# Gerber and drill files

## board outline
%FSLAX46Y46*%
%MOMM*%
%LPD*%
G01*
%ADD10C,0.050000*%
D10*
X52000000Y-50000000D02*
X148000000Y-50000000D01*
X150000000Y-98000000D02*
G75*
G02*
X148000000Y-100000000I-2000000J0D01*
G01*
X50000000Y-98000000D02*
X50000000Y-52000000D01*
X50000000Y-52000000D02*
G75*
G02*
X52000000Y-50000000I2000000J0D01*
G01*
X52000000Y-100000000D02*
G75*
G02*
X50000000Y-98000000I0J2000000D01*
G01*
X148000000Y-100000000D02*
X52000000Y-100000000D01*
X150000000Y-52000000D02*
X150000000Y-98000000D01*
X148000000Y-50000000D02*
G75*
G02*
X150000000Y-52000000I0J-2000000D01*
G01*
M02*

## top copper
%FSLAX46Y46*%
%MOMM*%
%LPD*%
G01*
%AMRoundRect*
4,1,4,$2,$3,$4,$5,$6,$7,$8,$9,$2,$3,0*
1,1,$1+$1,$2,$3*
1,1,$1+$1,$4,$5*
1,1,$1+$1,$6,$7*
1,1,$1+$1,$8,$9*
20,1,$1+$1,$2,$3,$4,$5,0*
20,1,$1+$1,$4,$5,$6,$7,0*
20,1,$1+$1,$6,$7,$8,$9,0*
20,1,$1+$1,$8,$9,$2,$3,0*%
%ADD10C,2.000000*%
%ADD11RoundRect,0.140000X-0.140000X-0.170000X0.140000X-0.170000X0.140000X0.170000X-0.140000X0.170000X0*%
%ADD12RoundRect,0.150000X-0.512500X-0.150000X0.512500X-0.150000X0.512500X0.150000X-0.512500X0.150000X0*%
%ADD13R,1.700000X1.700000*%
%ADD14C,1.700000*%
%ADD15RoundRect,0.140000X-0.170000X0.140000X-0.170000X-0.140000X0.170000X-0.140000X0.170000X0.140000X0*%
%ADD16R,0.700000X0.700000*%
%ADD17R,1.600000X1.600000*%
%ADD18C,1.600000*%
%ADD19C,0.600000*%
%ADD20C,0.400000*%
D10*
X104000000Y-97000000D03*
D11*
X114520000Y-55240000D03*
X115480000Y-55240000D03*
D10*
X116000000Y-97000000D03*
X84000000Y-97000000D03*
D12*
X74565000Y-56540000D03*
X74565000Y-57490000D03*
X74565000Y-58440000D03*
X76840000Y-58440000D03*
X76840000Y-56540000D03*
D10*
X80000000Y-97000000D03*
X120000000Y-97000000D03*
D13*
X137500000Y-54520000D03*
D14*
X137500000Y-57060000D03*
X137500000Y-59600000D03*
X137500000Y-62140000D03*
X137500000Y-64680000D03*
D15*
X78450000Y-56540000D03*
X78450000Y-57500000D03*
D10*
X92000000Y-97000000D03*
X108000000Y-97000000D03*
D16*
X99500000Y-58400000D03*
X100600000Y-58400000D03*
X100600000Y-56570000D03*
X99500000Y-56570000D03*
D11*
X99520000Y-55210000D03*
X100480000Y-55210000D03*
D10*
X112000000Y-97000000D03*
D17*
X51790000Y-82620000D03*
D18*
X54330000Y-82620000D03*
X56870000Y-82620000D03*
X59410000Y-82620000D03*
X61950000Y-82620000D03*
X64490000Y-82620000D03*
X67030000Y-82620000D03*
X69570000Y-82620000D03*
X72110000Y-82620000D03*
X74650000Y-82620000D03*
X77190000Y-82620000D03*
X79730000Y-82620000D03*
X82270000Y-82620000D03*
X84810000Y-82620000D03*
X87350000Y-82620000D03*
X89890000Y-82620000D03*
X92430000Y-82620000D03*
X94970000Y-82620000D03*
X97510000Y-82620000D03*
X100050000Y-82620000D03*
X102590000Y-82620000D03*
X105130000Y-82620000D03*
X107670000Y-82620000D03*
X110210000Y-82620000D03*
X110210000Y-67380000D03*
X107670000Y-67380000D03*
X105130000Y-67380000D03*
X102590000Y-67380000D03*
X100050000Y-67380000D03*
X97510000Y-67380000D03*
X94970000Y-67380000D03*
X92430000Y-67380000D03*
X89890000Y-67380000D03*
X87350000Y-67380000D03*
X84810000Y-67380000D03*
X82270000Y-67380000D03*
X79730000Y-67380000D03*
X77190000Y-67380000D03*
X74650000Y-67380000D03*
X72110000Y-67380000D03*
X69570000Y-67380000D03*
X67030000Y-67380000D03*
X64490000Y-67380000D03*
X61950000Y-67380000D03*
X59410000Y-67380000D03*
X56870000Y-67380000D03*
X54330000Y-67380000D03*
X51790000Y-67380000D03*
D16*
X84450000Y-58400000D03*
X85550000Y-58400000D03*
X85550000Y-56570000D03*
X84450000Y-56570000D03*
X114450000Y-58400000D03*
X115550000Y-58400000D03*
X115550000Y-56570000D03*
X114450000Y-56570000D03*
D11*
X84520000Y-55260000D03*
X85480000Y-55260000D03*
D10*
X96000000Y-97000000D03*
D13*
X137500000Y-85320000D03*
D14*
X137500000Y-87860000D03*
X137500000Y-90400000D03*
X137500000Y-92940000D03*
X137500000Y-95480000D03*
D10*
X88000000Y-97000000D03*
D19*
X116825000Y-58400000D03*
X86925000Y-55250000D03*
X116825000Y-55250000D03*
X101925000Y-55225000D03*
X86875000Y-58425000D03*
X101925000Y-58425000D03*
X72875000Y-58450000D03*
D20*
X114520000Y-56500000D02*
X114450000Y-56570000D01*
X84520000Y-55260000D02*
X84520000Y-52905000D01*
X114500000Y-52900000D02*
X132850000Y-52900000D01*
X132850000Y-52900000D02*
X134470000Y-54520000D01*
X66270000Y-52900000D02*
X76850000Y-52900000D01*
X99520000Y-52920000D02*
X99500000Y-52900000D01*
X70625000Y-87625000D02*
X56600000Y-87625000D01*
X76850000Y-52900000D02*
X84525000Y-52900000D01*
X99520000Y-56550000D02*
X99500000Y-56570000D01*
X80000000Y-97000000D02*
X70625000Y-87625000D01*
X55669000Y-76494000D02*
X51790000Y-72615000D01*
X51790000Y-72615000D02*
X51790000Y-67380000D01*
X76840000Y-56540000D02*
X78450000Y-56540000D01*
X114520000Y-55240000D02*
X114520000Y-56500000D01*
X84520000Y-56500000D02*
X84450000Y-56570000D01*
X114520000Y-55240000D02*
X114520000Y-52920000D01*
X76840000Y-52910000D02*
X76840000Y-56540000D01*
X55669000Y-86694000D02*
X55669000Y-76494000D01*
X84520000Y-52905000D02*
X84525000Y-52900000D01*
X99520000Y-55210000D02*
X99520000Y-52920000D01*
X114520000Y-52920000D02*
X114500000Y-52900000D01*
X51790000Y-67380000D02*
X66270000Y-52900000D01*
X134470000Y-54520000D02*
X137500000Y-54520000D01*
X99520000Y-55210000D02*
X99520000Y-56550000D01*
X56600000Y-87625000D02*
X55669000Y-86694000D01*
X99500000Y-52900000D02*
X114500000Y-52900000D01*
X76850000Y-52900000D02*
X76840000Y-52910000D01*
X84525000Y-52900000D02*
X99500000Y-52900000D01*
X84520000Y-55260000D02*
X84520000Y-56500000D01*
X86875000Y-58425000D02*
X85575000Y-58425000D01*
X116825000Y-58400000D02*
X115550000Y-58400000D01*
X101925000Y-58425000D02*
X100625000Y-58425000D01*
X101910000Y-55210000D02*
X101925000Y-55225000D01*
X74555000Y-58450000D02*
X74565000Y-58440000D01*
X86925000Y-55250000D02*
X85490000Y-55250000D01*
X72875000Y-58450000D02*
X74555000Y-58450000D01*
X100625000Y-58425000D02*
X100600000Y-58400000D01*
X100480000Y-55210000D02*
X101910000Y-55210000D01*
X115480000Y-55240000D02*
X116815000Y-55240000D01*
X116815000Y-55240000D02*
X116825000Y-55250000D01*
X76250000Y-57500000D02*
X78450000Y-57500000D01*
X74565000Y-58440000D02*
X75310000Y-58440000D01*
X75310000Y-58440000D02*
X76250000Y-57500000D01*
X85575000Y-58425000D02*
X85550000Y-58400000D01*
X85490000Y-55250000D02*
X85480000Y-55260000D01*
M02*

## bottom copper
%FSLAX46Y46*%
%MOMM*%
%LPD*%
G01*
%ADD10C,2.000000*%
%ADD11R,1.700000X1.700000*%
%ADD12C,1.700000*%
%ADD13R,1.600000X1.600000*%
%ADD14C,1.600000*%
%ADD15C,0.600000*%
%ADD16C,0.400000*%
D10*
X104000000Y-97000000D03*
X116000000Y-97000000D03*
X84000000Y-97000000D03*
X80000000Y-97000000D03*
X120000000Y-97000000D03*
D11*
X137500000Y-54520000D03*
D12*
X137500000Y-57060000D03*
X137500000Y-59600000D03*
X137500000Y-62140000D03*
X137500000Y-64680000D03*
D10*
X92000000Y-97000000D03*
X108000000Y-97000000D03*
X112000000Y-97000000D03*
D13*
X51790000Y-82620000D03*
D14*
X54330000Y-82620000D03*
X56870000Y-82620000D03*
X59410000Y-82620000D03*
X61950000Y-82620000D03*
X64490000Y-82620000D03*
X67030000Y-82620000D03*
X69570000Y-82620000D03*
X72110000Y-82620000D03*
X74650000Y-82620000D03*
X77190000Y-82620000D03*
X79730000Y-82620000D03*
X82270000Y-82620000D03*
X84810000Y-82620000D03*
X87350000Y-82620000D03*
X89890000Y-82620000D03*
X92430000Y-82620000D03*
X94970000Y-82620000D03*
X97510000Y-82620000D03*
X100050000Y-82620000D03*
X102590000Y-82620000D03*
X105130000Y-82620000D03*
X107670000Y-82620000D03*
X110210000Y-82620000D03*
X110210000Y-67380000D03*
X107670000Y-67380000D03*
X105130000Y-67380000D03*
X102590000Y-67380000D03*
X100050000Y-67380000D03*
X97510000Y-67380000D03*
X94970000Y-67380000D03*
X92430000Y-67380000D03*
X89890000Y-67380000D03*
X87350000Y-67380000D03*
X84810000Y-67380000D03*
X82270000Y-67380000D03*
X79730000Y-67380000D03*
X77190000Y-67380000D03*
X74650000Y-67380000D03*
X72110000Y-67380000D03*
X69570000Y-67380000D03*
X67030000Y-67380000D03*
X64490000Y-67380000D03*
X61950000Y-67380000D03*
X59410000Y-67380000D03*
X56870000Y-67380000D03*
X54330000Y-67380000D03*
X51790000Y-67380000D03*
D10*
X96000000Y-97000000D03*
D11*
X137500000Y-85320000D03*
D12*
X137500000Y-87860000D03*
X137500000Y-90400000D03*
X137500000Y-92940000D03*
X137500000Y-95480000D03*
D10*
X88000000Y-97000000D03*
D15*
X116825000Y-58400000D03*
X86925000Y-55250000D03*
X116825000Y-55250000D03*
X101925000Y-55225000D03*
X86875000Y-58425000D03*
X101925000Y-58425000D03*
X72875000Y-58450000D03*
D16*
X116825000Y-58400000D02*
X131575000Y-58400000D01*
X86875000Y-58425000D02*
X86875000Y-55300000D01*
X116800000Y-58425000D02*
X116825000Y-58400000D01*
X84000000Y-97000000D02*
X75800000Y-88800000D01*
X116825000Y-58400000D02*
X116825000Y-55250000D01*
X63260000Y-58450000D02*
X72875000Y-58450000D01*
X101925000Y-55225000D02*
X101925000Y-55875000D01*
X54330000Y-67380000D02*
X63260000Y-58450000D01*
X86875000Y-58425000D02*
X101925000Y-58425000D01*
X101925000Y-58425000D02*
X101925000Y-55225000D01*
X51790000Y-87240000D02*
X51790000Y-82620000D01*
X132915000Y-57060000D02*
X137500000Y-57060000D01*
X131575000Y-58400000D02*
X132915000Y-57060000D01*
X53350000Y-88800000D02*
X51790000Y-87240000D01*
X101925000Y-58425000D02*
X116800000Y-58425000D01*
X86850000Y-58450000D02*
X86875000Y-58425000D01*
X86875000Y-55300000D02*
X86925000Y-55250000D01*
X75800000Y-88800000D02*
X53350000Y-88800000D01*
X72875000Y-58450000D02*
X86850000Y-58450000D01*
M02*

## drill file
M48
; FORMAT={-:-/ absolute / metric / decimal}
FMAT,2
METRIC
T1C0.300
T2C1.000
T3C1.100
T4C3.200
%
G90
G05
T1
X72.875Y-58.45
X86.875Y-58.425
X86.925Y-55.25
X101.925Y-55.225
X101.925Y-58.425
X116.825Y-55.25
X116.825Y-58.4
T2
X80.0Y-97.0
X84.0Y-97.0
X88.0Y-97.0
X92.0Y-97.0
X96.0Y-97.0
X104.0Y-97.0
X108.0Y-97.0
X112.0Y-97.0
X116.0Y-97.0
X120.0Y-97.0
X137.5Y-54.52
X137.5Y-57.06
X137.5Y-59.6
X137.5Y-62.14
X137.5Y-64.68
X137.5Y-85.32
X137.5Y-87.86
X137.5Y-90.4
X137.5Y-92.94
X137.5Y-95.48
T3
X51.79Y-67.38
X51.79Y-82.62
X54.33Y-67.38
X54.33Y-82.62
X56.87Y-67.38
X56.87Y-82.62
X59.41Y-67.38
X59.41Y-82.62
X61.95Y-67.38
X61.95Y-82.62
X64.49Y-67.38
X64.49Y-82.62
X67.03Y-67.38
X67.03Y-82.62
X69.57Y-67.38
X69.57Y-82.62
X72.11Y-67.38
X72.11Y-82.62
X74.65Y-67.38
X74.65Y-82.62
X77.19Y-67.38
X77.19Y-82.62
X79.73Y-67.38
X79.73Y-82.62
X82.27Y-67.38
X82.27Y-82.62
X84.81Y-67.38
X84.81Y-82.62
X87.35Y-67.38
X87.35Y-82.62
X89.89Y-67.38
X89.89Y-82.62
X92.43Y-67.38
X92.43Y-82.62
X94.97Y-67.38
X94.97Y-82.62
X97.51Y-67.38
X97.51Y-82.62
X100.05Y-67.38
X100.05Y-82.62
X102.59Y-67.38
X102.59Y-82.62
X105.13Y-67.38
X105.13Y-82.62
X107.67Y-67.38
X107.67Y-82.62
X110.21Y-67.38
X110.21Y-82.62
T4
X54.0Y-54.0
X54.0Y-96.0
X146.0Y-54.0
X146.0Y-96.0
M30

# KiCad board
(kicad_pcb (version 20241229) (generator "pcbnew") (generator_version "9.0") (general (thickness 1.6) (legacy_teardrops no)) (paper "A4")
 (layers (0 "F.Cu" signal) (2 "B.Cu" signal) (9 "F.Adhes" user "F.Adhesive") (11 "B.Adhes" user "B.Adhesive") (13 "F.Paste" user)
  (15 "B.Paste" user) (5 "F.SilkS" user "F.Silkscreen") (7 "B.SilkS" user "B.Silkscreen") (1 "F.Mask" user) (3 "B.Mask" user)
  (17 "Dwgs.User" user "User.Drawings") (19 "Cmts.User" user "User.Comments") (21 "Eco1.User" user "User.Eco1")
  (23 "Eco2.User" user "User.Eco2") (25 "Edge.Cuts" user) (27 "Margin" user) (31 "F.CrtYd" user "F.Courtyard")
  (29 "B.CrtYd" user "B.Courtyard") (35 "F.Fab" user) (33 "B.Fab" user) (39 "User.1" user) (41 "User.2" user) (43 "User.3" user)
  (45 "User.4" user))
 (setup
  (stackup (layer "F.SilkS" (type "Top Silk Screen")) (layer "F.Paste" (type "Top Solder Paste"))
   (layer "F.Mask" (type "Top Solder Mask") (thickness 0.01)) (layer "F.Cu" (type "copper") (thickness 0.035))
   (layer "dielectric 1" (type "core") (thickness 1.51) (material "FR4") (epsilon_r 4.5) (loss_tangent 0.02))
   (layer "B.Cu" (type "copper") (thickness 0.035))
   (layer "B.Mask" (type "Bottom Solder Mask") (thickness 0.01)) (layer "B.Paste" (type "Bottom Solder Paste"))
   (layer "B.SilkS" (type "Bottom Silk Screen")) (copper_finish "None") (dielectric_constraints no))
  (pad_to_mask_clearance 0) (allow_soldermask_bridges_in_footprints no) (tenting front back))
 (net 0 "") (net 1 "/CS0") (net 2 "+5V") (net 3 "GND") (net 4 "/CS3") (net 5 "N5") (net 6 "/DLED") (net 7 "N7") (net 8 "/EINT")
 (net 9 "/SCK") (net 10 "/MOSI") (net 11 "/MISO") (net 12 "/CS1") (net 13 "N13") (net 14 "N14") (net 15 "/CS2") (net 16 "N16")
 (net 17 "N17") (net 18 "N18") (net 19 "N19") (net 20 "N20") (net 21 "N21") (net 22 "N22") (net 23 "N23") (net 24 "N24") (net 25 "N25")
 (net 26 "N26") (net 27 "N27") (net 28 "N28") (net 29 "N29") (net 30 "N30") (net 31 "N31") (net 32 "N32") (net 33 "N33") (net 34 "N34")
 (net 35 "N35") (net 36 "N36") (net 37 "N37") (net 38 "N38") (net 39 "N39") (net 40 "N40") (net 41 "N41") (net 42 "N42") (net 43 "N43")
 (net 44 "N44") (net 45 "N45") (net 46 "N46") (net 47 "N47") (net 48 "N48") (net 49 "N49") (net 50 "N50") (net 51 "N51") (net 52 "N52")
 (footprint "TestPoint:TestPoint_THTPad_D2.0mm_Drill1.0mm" (layer "F.Cu") (at 104 97 90)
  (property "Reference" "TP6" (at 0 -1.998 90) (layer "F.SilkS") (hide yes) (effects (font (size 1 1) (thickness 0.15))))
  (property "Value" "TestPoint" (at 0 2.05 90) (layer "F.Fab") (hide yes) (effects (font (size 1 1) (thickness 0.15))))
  (pad "1" thru_hole circle (at 0 0 90) (size 2 2) (drill 1) (layers "*.Cu" "*.Mask") (remove_unused_layers no) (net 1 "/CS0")))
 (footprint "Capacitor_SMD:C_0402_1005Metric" (layer "F.Cu") (at 115 55.24)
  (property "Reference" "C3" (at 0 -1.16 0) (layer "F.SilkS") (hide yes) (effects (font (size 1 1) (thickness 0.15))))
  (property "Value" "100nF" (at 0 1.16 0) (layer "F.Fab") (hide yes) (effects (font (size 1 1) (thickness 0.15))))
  (pad "1" smd roundrect (at -0.48 0) (size 0.56 0.62) (layers "F.Cu" "F.Mask" "F.Paste") (roundrect_rratio 0.25) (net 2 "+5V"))
  (pad "2" smd roundrect (at 0.48 0) (size 0.56 0.62) (layers "F.Cu" "F.Mask" "F.Paste") (roundrect_rratio 0.25) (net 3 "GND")))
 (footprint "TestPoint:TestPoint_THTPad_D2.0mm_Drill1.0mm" (layer "F.Cu") (at 116 97 90)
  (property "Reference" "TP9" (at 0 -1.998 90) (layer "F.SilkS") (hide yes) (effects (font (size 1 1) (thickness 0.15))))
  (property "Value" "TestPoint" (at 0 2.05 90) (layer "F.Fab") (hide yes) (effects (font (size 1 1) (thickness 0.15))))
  (pad "1" thru_hole circle (at 0 0 90) (size 2 2) (drill 1) (layers "*.Cu" "*.Mask") (remove_unused_layers no) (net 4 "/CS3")))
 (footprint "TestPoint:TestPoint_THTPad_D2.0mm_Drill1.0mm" (layer "F.Cu") (at 84 97 90)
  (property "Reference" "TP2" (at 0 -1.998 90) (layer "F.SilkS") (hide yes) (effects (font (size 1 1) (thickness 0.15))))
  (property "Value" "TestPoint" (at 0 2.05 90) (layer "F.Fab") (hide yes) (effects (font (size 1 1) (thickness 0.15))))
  (pad "1" thru_hole circle (at 0 0 90) (size 2 2) (drill 1) (layers "*.Cu" "*.Mask") (remove_unused_layers no) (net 3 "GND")))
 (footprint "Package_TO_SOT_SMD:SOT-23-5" (layer "F.Cu") (at 75.7025 57.49)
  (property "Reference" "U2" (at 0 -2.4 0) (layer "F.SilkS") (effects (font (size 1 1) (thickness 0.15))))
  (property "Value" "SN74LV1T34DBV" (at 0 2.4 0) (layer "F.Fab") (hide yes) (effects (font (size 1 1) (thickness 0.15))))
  (pad "1" smd roundrect (at -1.1375 -0.95) (size 1.325 0.6) (layers "F.Cu" "F.Mask" "F.Paste") (roundrect_rratio 0.25) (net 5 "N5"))
  (pad "2" smd roundrect (at -1.1375 0) (size 1.325 0.6) (layers "F.Cu" "F.Mask" "F.Paste") (roundrect_rratio 0.25) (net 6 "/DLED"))
  (pad "3" smd roundrect (at -1.1375 0.95) (size 1.325 0.6) (layers "F.Cu" "F.Mask" "F.Paste") (roundrect_rratio 0.25) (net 3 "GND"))
  (pad "4" smd roundrect (at 1.1375 0.95) (size 1.325 0.6) (layers "F.Cu" "F.Mask" "F.Paste") (roundrect_rratio 0.25) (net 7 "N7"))
  (pad "5" smd roundrect (at 1.1375 -0.95) (size 1.325 0.6) (layers "F.Cu" "F.Mask" "F.Paste") (roundrect_rratio 0.25) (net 2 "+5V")))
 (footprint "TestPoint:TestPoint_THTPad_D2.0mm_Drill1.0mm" (layer "F.Cu") (at 80 97 90)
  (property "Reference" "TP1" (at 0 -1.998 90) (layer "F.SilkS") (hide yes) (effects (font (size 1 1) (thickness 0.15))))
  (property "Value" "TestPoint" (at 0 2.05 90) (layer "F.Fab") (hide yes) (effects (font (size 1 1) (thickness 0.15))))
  (pad "1" thru_hole circle (at 0 0 90) (size 2 2) (drill 1) (layers "*.Cu" "*.Mask") (remove_unused_layers no) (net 2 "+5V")))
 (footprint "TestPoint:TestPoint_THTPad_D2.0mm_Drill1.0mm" (layer "F.Cu") (at 120 97 90)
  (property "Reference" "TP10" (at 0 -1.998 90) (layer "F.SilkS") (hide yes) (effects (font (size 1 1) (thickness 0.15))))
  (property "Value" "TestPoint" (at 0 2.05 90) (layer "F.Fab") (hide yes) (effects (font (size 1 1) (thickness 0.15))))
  (pad "1" thru_hole circle (at 0 0 90) (size 2 2) (drill 1) (layers "*.Cu" "*.Mask") (remove_unused_layers no) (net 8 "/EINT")))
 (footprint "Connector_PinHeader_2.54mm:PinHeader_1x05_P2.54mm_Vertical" (layer "F.Cu") (at 137.5 54.52)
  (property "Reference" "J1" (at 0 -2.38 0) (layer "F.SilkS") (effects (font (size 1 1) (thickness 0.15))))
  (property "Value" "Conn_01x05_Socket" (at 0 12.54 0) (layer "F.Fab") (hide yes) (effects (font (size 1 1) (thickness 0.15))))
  (pad "1" thru_hole rect (at 0 0) (size 1.7 1.7) (drill 1) (layers "*.Cu" "*.Mask") (remove_unused_layers no) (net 2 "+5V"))
  (pad "2" thru_hole circle (at 0 2.54) (size 1.7 1.7) (drill 1) (layers "*.Cu" "*.Mask") (remove_unused_layers no) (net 3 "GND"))
  (pad "3" thru_hole circle (at 0 5.08) (size 1.7 1.7) (drill 1) (layers "*.Cu" "*.Mask") (remove_unused_layers no) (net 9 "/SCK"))
  (pad "4" thru_hole circle (at 0 7.62) (size 1.7 1.7) (drill 1) (layers "*.Cu" "*.Mask") (remove_unused_layers no) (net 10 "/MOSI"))
  (pad "5" thru_hole circle (at 0 10.16) (size 1.7 1.7) (drill 1) (layers "*.Cu" "*.Mask") (remove_unused_layers no) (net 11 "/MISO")))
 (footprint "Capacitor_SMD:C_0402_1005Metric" (layer "F.Cu") (at 78.45 57.02 -90)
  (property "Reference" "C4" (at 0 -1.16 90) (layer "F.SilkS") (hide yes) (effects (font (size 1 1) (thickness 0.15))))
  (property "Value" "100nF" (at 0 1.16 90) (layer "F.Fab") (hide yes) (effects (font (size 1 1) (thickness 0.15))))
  (pad "1" smd roundrect (at -0.48 0 270) (size 0.56 0.62) (layers "F.Cu" "F.Mask" "F.Paste") (roundrect_rratio 0.25) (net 2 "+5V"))
  (pad "2" smd roundrect (at 0.48 0 270) (size 0.56 0.62) (layers "F.Cu" "F.Mask" "F.Paste") (roundrect_rratio 0.25) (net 3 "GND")))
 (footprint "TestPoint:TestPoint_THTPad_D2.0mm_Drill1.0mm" (layer "F.Cu") (at 92 97 90)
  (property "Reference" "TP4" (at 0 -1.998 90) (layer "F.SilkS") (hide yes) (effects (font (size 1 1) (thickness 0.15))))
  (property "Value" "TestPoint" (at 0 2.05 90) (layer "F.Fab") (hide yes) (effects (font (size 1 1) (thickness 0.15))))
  (pad "1" thru_hole circle (at 0 0 90) (size 2 2) (drill 1) (layers "*.Cu" "*.Mask") (remove_unused_layers no) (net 10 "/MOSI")))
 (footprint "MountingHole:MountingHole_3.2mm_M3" (layer "F.Cu") (at 54 96)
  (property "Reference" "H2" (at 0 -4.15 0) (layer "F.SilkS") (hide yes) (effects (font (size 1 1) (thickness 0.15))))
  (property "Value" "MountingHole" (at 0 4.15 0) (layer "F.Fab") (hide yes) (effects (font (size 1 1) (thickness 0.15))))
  (pad "" np_thru_hole circle (at 0 0) (size 3.2 3.2) (drill 3.2) (layers "*.Cu" "*.Mask")))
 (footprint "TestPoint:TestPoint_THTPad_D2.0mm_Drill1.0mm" (layer "F.Cu") (at 108 97 90)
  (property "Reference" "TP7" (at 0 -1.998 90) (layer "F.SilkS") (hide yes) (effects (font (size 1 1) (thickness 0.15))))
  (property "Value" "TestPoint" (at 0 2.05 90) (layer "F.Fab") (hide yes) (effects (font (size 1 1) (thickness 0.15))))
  (pad "1" thru_hole circle (at 0 0 90) (size 2 2) (drill 1) (layers "*.Cu" "*.Mask") (remove_unused_layers no) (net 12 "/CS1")))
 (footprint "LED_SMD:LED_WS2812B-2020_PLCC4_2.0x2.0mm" (layer "F.Cu") (at 100.05 57.485 90)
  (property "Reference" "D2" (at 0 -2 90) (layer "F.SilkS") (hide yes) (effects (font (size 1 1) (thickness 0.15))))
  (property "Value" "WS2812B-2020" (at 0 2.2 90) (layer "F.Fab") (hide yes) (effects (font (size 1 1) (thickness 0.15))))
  (pad "1" smd rect (at -0.915 -0.55 90) (size 0.7 0.7) (layers "F.Cu" "F.Mask" "F.Paste") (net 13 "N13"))
  (pad "2" smd rect (at -0.915 0.55 90) (size 0.7 0.7) (layers "F.Cu" "F.Mask" "F.Paste") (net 3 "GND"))
  (pad "3" smd rect (at 0.915 0.55 90) (size 0.7 0.7) (layers "F.Cu" "F.Mask" "F.Paste") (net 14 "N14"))
  (pad "4" smd rect (at 0.915 -0.55 90) (size 0.7 0.7) (layers "F.Cu" "F.Mask" "F.Paste") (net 2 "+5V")))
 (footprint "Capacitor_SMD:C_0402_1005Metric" (layer "F.Cu") (at 100 55.21)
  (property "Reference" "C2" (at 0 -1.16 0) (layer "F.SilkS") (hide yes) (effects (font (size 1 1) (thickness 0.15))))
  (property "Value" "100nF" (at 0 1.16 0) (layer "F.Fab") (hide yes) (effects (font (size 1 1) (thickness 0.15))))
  (pad "1" smd roundrect (at -0.48 0) (size 0.56 0.62) (layers "F.Cu" "F.Mask" "F.Paste") (roundrect_rratio 0.25) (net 2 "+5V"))
  (pad "2" smd roundrect (at 0.48 0) (size 0.56 0.62) (layers "F.Cu" "F.Mask" "F.Paste") (roundrect_rratio 0.25) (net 3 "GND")))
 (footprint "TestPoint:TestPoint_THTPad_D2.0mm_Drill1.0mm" (layer "F.Cu") (at 112 97 90)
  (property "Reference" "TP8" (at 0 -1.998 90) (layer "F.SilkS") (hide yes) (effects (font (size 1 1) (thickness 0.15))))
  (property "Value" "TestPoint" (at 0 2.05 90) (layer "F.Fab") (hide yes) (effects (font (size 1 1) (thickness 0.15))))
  (pad "1" thru_hole circle (at 0 0 90) (size 2 2) (drill 1) (layers "*.Cu" "*.Mask") (remove_unused_layers no) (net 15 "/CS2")))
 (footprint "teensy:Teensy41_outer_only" (layer "F.Cu") (at 81 75)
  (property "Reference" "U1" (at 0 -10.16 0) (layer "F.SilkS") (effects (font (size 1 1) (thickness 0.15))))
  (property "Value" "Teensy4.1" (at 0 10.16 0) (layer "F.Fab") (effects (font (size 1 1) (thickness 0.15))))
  (pad "1" thru_hole rect (at -29.21 7.62) (size 1.6 1.6) (drill 1.1) (layers "*.Cu" "*.Mask") (remove_unused_layers no) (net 3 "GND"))
  (pad "2" thru_hole circle (at -26.67 7.62) (size 1.6 1.6) (drill 1.1) (layers "*.Cu" "*.Mask") (remove_unused_layers no) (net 1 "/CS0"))
  (pad "3" thru_hole circle (at -24.13 7.62) (size 1.6 1.6) (drill 1.1) (layers "*.Cu" "*.Mask") (remove_unused_layers no) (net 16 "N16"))
  (pad "4" thru_hole circle (at -21.59 7.62) (size 1.6 1.6) (drill 1.1) (layers "*.Cu" "*.Mask") (remove_unused_layers no) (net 12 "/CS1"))
  (pad "5" thru_hole circle (at -19.05 7.62) (size 1.6 1.6) (drill 1.1) (layers "*.Cu" "*.Mask") (remove_unused_layers no) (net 15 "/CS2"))
  (pad "6" thru_hole circle (at -16.51 7.62) (size 1.6 1.6) (drill 1.1) (layers "*.Cu" "*.Mask") (remove_unused_layers no) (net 4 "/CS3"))
  (pad "7" thru_hole circle (at -13.97 7.62) (size 1.6 1.6) (drill 1.1) (layers "*.Cu" "*.Mask") (remove_unused_layers no) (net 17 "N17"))
  (pad "8" thru_hole circle (at -11.43 7.62) (size 1.6 1.6) (drill 1.1) (layers "*.Cu" "*.Mask") (remove_unused_layers no) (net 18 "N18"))
  (pad "9" thru_hole circle (at -8.89 7.62) (size 1.6 1.6) (drill 1.1) (layers "*.Cu" "*.Mask") (remove_unused_layers no) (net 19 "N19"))
  (pad "10" thru_hole circle (at -6.35 7.62) (size 1.6 1.6) (drill 1.1) (layers "*.Cu" "*.Mask") (remove_unused_layers no) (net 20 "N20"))
  (pad "11" thru_hole circle (at -3.81 7.62) (size 1.6 1.6) (drill 1.1) (layers "*.Cu" "*.Mask") (remove_unused_layers no) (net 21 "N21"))
  (pad "12" thru_hole circle (at -1.27 7.62) (size 1.6 1.6) (drill 1.1) (layers "*.Cu" "*.Mask") (remove_unused_layers no) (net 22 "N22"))
  (pad "13" thru_hole circle (at 1.27 7.62) (size 1.6 1.6) (drill 1.1) (layers "*.Cu" "*.Mask") (remove_unused_layers no) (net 10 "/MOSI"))
  (pad "14" thru_hole circle (at 3.81 7.62) (size 1.6 1.6) (drill 1.1) (layers "*.Cu" "*.Mask") (remove_unused_layers no) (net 11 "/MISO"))
  (pad "15" thru_hole circle (at 6.35 7.62) (size 1.6 1.6) (drill 1.1) (layers "*.Cu" "*.Mask") (remove_unused_layers no) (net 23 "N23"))
  (pad "16" thru_hole circle (at 8.89 7.62) (size 1.6 1.6) (drill 1.1) (layers "*.Cu" "*.Mask") (remove_unused_layers no) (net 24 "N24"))
  (pad "17" thru_hole circle (at 11.43 7.62) (size 1.6 1.6) (drill 1.1) (layers "*.Cu" "*.Mask") (remove_unused_layers no) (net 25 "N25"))
  (pad "18" thru_hole circle (at 13.97 7.62) (size 1.6 1.6) (drill 1.1) (layers "*.Cu" "*.Mask") (remove_unused_layers no) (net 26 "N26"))
  (pad "19" thru_hole circle (at 16.51 7.62) (size 1.6 1.6) (drill 1.1) (layers "*.Cu" "*.Mask") (remove_unused_layers no) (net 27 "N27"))
  (pad "20" thru_hole circle (at 19.05 7.62) (size 1.6 1.6) (drill 1.1) (layers "*.Cu" "*.Mask") (remove_unused_layers no) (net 6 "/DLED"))
  (pad "21" thru_hole circle (at 21.59 7.62) (size 1.6 1.6) (drill 1.1) (layers "*.Cu" "*.Mask") (remove_unused_layers no) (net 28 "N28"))
  (pad "22" thru_hole circle (at 24.13 7.62) (size 1.6 1.6) (drill 1.1) (layers "*.Cu" "*.Mask") (remove_unused_layers no) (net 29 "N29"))
  (pad "23" thru_hole circle (at 26.67 7.62) (size 1.6 1.6) (drill 1.1) (layers "*.Cu" "*.Mask") (remove_unused_layers no) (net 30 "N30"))
  (pad "24" thru_hole circle (at 29.21 7.62) (size 1.6 1.6) (drill 1.1) (layers "*.Cu" "*.Mask") (remove_unused_layers no) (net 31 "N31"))
  (pad "25" thru_hole circle (at 29.21 -7.62) (size 1.6 1.6) (drill 1.1) (layers "*.Cu" "*.Mask") (remove_unused_layers no) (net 8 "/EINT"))
  (pad "26" thru_hole circle (at 26.67 -7.62) (size 1.6 1.6) (drill 1.1) (layers "*.Cu" "*.Mask") (remove_unused_layers no) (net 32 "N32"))
  (pad "27" thru_hole circle (at 24.13 -7.62) (size 1.6 1.6) (drill 1.1) (layers "*.Cu" "*.Mask") (remove_unused_layers no) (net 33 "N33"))
  (pad "28" thru_hole circle (at 21.59 -7.62) (size 1.6 1.6) (drill 1.1) (layers "*.Cu" "*.Mask") (remove_unused_layers no) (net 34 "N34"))
  (pad "29" thru_hole circle (at 19.05 -7.62) (size 1.6 1.6) (drill 1.1) (layers "*.Cu" "*.Mask") (remove_unused_layers no) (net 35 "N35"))
  (pad "30" thru_hole circle (at 16.51 -7.62) (size 1.6 1.6) (drill 1.1) (layers "*.Cu" "*.Mask") (remove_unused_layers no) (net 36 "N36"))
  (pad "31" thru_hole circle (at 13.97 -7.62) (size 1.6 1.6) (drill 1.1) (layers "*.Cu" "*.Mask") (remove_unused_layers no) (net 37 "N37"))
  (pad "32" thru_hole circle (at 11.43 -7.62) (size 1.6 1.6) (drill 1.1) (layers "*.Cu" "*.Mask") (remove_unused_layers no) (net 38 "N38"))
  (pad "33" thru_hole circle (at 8.89 -7.62) (size 1.6 1.6) (drill 1.1) (layers "*.Cu" "*.Mask") (remove_unused_layers no) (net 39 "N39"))
  (pad "34" thru_hole circle (at 6.35 -7.62) (size 1.6 1.6) (drill 1.1) (layers "*.Cu" "*.Mask") (remove_unused_layers no) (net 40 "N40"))
  (pad "35" thru_hole circle (at 3.81 -7.62) (size 1.6 1.6) (drill 1.1) (layers "*.Cu" "*.Mask") (remove_unused_layers no) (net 9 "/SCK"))
  (pad "36" thru_hole circle (at 1.27 -7.62) (size 1.6 1.6) (drill 1.1) (layers "*.Cu" "*.Mask") (remove_unused_layers no) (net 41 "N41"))
  (pad "37" thru_hole circle (at -1.27 -7.62) (size 1.6 1.6) (drill 1.1) (layers "*.Cu" "*.Mask") (remove_unused_layers no) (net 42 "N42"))
  (pad "38" thru_hole circle (at -3.81 -7.62) (size 1.6 1.6) (drill 1.1) (layers "*.Cu" "*.Mask") (remove_unused_layers no) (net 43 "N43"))
  (pad "39" thru_hole circle (at -6.35 -7.62) (size 1.6 1.6) (drill 1.1) (layers "*.Cu" "*.Mask") (remove_unused_layers no) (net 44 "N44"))
  (pad "40" thru_hole circle (at -8.89 -7.62) (size 1.6 1.6) (drill 1.1) (layers "*.Cu" "*.Mask") (remove_unused_layers no) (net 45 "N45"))
  (pad "41" thru_hole circle (at -11.43 -7.62) (size 1.6 1.6) (drill 1.1) (layers "*.Cu" "*.Mask") (remove_unused_layers no) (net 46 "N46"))
  (pad "42" thru_hole circle (at -13.97 -7.62) (size 1.6 1.6) (drill 1.1) (layers "*.Cu" "*.Mask") (remove_unused_layers no) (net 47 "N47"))
  (pad "43" thru_hole circle (at -16.51 -7.62) (size 1.6 1.6) (drill 1.1) (layers "*.Cu" "*.Mask") (remove_unused_layers no) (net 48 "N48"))
  (pad "44" thru_hole circle (at -19.05 -7.62) (size 1.6 1.6) (drill 1.1) (layers "*.Cu" "*.Mask") (remove_unused_layers no) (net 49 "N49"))
  (pad "45" thru_hole circle (at -21.59 -7.62) (size 1.6 1.6) (drill 1.1) (layers "*.Cu" "*.Mask") (remove_unused_layers no) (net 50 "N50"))
  (pad "46" thru_hole circle (at -24.13 -7.62) (size 1.6 1.6) (drill 1.1) (layers "*.Cu" "*.Mask") (remove_unused_layers no) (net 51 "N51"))
  (pad "47" thru_hole circle (at -26.67 -7.62) (size 1.6 1.6) (drill 1.1) (layers "*.Cu" "*.Mask") (remove_unused_layers no) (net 3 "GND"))
  (pad "48" thru_hole circle (at -29.21 -7.62) (size 1.6 1.6) (drill 1.1) (layers "*.Cu" "*.Mask") (remove_unused_layers no) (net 2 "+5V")))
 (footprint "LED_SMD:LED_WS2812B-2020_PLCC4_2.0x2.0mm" (layer "F.Cu") (at 85 57.485 90)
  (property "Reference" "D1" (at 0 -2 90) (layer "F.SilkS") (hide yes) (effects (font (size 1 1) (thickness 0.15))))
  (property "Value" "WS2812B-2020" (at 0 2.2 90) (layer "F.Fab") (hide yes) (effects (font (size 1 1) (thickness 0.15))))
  (pad "1" smd rect (at -0.915 -0.55 90) (size 0.7 0.7) (layers "F.Cu" "F.Mask" "F.Paste") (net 14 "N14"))
  (pad "2" smd rect (at -0.915 0.55 90) (size 0.7 0.7) (layers "F.Cu" "F.Mask" "F.Paste") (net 3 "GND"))
  (pad "3" smd rect (at 0.915 0.55 90) (size 0.7 0.7) (layers "F.Cu" "F.Mask" "F.Paste") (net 7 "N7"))
  (pad "4" smd rect (at 0.915 -0.55 90) (size 0.7 0.7) (layers "F.Cu" "F.Mask" "F.Paste") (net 2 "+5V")))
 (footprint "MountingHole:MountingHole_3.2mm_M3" (layer "F.Cu") (at 146 96)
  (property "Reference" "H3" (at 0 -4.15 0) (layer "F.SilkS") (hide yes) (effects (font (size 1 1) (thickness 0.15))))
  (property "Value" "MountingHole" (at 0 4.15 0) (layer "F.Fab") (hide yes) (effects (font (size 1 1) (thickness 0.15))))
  (pad "" np_thru_hole circle (at 0 0) (size 3.2 3.2) (drill 3.2) (layers "*.Cu" "*.Mask")))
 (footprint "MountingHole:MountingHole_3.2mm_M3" (layer "F.Cu") (at 146 54)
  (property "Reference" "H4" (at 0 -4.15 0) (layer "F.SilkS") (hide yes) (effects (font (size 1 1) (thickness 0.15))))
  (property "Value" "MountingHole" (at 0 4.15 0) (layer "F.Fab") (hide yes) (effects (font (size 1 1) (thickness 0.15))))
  (pad "" np_thru_hole circle (at 0 0) (size 3.2 3.2) (drill 3.2) (layers "*.Cu" "*.Mask")))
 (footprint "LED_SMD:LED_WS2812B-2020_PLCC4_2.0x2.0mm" (layer "F.Cu") (at 115 57.485 90)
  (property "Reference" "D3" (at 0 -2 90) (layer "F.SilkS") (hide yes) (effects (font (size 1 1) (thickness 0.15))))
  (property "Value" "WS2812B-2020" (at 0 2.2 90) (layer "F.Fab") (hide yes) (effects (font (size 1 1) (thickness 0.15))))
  (pad "1" smd rect (at -0.915 -0.55 90) (size 0.7 0.7) (layers "F.Cu" "F.Mask" "F.Paste") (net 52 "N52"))
  (pad "2" smd rect (at -0.915 0.55 90) (size 0.7 0.7) (layers "F.Cu" "F.Mask" "F.Paste") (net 3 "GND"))
  (pad "3" smd rect (at 0.915 0.55 90) (size 0.7 0.7) (layers "F.Cu" "F.Mask" "F.Paste") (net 13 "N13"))
  (pad "4" smd rect (at 0.915 -0.55 90) (size 0.7 0.7) (layers "F.Cu" "F.Mask" "F.Paste") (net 2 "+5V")))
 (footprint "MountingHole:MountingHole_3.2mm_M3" (layer "F.Cu") (at 54 54)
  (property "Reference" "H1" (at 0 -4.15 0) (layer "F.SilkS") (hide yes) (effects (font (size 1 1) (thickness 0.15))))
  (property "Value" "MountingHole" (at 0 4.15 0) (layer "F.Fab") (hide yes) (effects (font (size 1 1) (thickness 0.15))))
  (pad "" np_thru_hole circle (at 0 0) (size 3.2 3.2) (drill 3.2) (layers "*.Cu" "*.Mask")))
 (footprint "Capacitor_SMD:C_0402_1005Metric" (layer "F.Cu") (at 85 55.26)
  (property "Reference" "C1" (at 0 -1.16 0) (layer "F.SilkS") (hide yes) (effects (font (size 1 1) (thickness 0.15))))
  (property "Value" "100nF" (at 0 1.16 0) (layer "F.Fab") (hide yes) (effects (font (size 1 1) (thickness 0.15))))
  (pad "1" smd roundrect (at -0.48 0) (size 0.56 0.62) (layers "F.Cu" "F.Mask" "F.Paste") (roundrect_rratio 0.25) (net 2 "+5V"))
  (pad "2" smd roundrect (at 0.48 0) (size 0.56 0.62) (layers "F.Cu" "F.Mask" "F.Paste") (roundrect_rratio 0.25) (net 3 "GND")))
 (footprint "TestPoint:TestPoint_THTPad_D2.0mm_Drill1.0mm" (layer "F.Cu") (at 96 97 90)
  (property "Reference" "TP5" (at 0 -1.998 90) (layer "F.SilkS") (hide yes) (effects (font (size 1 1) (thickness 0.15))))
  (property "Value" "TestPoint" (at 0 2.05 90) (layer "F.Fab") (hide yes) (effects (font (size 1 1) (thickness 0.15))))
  (pad "1" thru_hole circle (at 0 0 90) (size 2 2) (drill 1) (layers "*.Cu" "*.Mask") (remove_unused_layers no) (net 11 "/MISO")))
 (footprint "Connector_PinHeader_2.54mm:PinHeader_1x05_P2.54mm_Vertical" (layer "F.Cu") (at 137.5 85.32)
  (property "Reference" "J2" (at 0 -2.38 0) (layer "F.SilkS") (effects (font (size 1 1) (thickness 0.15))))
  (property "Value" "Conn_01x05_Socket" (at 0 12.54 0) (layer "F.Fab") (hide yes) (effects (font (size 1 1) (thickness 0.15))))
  (pad "1" thru_hole rect (at 0 0) (size 1.7 1.7) (drill 1) (layers "*.Cu" "*.Mask") (remove_unused_layers no) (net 1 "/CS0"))
  (pad "2" thru_hole circle (at 0 2.54) (size 1.7 1.7) (drill 1) (layers "*.Cu" "*.Mask") (remove_unused_layers no) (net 12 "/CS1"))
  (pad "3" thru_hole circle (at 0 5.08) (size 1.7 1.7) (drill 1) (layers "*.Cu" "*.Mask") (remove_unused_layers no) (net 15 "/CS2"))
  (pad "4" thru_hole circle (at 0 7.62) (size 1.7 1.7) (drill 1) (layers "*.Cu" "*.Mask") (remove_unused_layers no) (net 4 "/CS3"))
  (pad "5" thru_hole circle (at 0 10.16) (size 1.7 1.7) (drill 1) (layers "*.Cu" "*.Mask") (remove_unused_layers no) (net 8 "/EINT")))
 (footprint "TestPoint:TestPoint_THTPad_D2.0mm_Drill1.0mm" (layer "F.Cu") (at 88 97 90)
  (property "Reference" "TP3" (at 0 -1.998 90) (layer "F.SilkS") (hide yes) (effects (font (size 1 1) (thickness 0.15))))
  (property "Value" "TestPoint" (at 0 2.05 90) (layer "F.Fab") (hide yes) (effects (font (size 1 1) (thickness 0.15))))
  (pad "1" thru_hole circle (at 0 0 90) (size 2 2) (drill 1) (layers "*.Cu" "*.Mask") (remove_unused_layers no) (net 9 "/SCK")))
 (gr_line (start 52 50) (end 148 50) (stroke (width 0.05) (type default)) (layer "Edge.Cuts"))
 (gr_arc (start 150 98) (mid 149.414214 99.414214) (end 148 100) (stroke (width 0.05) (type default)) (layer "Edge.Cuts"))
 (gr_line (start 50 98) (end 50 52) (stroke (width 0.05) (type default)) (layer "Edge.Cuts"))
 (gr_arc (start 50 52) (mid 50.585786 50.585786) (end 52 50) (stroke (width 0.05) (type default)) (layer "Edge.Cuts"))
 (gr_arc (start 52 100) (mid 50.585786 99.414214) (end 50 98) (stroke (width 0.05) (type default)) (layer "Edge.Cuts"))
 (gr_line (start 148 100) (end 52 100) (stroke (width 0.05) (type default)) (layer "Edge.Cuts"))
 (gr_line (start 150 52) (end 150 98) (stroke (width 0.05) (type default)) (layer "Edge.Cuts"))
 (gr_arc (start 148 50) (mid 149.414214 50.585786) (end 150 52) (stroke (width 0.05) (type default)) (layer "Edge.Cuts"))
 (segment (start 114.52 56.5) (end 114.45 56.57) (width 0.4) (layer "F.Cu") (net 2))
 (segment (start 84.52 55.26) (end 84.52 52.905) (width 0.4) (layer "F.Cu") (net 2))
 (segment (start 114.5 52.9) (end 132.85 52.9) (width 0.4) (layer "F.Cu") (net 2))
 (segment (start 132.85 52.9) (end 134.47 54.52) (width 0.4) (layer "F.Cu") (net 2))
 (segment (start 66.27 52.9) (end 76.85 52.9) (width 0.4) (layer "F.Cu") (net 2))
 (segment (start 99.52 52.92) (end 99.5 52.9) (width 0.4) (layer "F.Cu") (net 2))
 (segment (start 70.625 87.625) (end 56.6 87.625) (width 0.4) (layer "F.Cu") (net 2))
 (segment (start 76.85 52.9) (end 84.525 52.9) (width 0.4) (layer "F.Cu") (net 2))
 (segment (start 99.52 56.55) (end 99.5 56.57) (width 0.4) (layer "F.Cu") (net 2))
 (segment (start 80 97) (end 70.625 87.625) (width 0.4) (layer "F.Cu") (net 2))
 (segment (start 55.669 76.494) (end 51.79 72.615) (width 0.4) (layer "F.Cu") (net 2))
 (segment (start 51.79 72.615) (end 51.79 67.38) (width 0.4) (layer "F.Cu") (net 2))
 (segment (start 76.84 56.54) (end 78.45 56.54) (width 0.4) (layer "F.Cu") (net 2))
 (segment (start 114.52 55.24) (end 114.52 56.5) (width 0.4) (layer "F.Cu") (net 2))
 (segment (start 84.52 56.5) (end 84.45 56.57) (width 0.4) (layer "F.Cu") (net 2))
 (segment (start 114.52 55.24) (end 114.52 52.92) (width 0.4) (layer "F.Cu") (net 2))
 (segment (start 76.84 52.91) (end 76.84 56.54) (width 0.4) (layer "F.Cu") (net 2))
 (segment (start 55.669 86.694) (end 55.669 76.494) (width 0.4) (layer "F.Cu") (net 2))
 (segment (start 84.52 52.905) (end 84.525 52.9) (width 0.4) (layer "F.Cu") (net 2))
 (segment (start 99.52 55.21) (end 99.52 52.92) (width 0.4) (layer "F.Cu") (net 2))
 (segment (start 114.52 52.92) (end 114.5 52.9) (width 0.4) (layer "F.Cu") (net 2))
 (segment (start 51.79 67.38) (end 66.27 52.9) (width 0.4) (layer "F.Cu") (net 2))
 (segment (start 134.47 54.52) (end 137.5 54.52) (width 0.4) (layer "F.Cu") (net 2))
 (segment (start 99.52 55.21) (end 99.52 56.55) (width 0.4) (layer "F.Cu") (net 2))
 (segment (start 56.6 87.625) (end 55.669 86.694) (width 0.4) (layer "F.Cu") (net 2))
 (segment (start 99.5 52.9) (end 114.5 52.9) (width 0.4) (layer "F.Cu") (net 2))
 (segment (start 76.85 52.9) (end 76.84 52.91) (width 0.4) (layer "F.Cu") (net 2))
 (segment (start 84.525 52.9) (end 99.5 52.9) (width 0.4) (layer "F.Cu") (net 2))
 (segment (start 84.52 55.26) (end 84.52 56.5) (width 0.4) (layer "F.Cu") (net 2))
 (segment (start 86.875 58.425) (end 85.575 58.425) (width 0.4) (layer "F.Cu") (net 3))
 (segment (start 116.825 58.4) (end 115.55 58.4) (width 0.4) (layer "F.Cu") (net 3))
 (segment (start 101.925 58.425) (end 100.625 58.425) (width 0.4) (layer "F.Cu") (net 3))
 (segment (start 101.91 55.21) (end 101.925 55.225) (width 0.4) (layer "F.Cu") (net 3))
 (segment (start 74.555 58.45) (end 74.565 58.44) (width 0.4) (layer "F.Cu") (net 3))
 (segment (start 86.925 55.25) (end 85.49 55.25) (width 0.4) (layer "F.Cu") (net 3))
 (segment (start 72.875 58.45) (end 74.555 58.45) (width 0.4) (layer "F.Cu") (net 3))
 (segment (start 100.625 58.425) (end 100.6 58.4) (width 0.4) (layer "F.Cu") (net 3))
 (segment (start 100.48 55.21) (end 101.91 55.21) (width 0.4) (layer "F.Cu") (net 3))
 (segment (start 115.48 55.24) (end 116.815 55.24) (width 0.4) (layer "F.Cu") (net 3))
 (segment (start 116.815 55.24) (end 116.825 55.25) (width 0.4) (layer "F.Cu") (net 3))
 (segment (start 76.25 57.5) (end 78.45 57.5) (width 0.4) (layer "F.Cu") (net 3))
 (segment (start 74.565 58.44) (end 75.31 58.44) (width 0.4) (layer "F.Cu") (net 3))
 (segment (start 75.31 58.44) (end 76.25 57.5) (width 0.4) (layer "F.Cu") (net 3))
 (segment (start 85.575 58.425) (end 85.55 58.4) (width 0.4) (layer "F.Cu") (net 3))
 (segment (start 85.49 55.25) (end 85.48 55.26) (width 0.4) (layer "F.Cu") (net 3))
 (via (at 116.825 58.4) (size 0.6) (drill 0.3) (layers "F.Cu" "B.Cu") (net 3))
 (via (at 86.925 55.25) (size 0.6) (drill 0.3) (layers "F.Cu" "B.Cu") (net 3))
 (via (at 116.825 55.25) (size 0.6) (drill 0.3) (layers "F.Cu" "B.Cu") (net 3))
 (via (at 101.925 55.225) (size 0.6) (drill 0.3) (layers "F.Cu" "B.Cu") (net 3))
 (via (at 86.875 58.425) (size 0.6) (drill 0.3) (layers "F.Cu" "B.Cu") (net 3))
 (via (at 101.925 58.425) (size 0.6) (drill 0.3) (layers "F.Cu" "B.Cu") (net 3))
 (via (at 72.875 58.45) (size 0.6) (drill 0.3) (layers "F.Cu" "B.Cu") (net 3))
 (segment (start 116.825 58.4) (end 131.575 58.4) (width 0.4) (layer "B.Cu") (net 3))
 (segment (start 86.875 58.425) (end 86.875 55.3) (width 0.4) (layer "B.Cu") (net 3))
 (segment (start 116.8 58.425) (end 116.825 58.4) (width 0.4) (layer "B.Cu") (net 3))
 (segment (start 84 97) (end 75.8 88.8) (width 0.4) (layer "B.Cu") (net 3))
 (segment (start 116.825 58.4) (end 116.825 55.25) (width 0.4) (layer "B.Cu") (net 3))
 (segment (start 63.26 58.45) (end 72.875 58.45) (width 0.4) (layer "B.Cu") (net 3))
 (segment (start 101.925 55.225) (end 101.925 55.875) (width 0.4) (layer "B.Cu") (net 3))
 (segment (start 54.33 67.38) (end 63.26 58.45) (width 0.4) (layer "B.Cu") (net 3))
 (segment (start 86.875 58.425) (end 101.925 58.425) (width 0.4) (layer "B.Cu") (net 3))
 (segment (start 101.925 58.425) (end 101.925 55.225) (width 0.4) (layer "B.Cu") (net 3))
 (segment (start 51.79 87.24) (end 51.79 82.62) (width 0.4) (layer "B.Cu") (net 3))
 (segment (start 132.915 57.06) (end 137.5 57.06) (width 0.4) (layer "B.Cu") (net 3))
 (segment (start 131.575 58.4) (end 132.915 57.06) (width 0.4) (layer "B.Cu") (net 3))
 (segment (start 53.35 88.8) (end 51.79 87.24) (width 0.4) (layer "B.Cu") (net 3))
 (segment (start 101.925 58.425) (end 116.8 58.425) (width 0.4) (layer "B.Cu") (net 3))
 (segment (start 86.85 58.45) (end 86.875 58.425) (width 0.4) (layer "B.Cu") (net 3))
 (segment (start 86.875 55.3) (end 86.925 55.25) (width 0.4) (layer "B.Cu") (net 3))
 (segment (start 75.8 88.8) (end 53.35 88.8) (width 0.4) (layer "B.Cu") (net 3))
 (segment (start 72.875 58.45) (end 86.85 58.45) (width 0.4) (layer "B.Cu") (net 3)))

